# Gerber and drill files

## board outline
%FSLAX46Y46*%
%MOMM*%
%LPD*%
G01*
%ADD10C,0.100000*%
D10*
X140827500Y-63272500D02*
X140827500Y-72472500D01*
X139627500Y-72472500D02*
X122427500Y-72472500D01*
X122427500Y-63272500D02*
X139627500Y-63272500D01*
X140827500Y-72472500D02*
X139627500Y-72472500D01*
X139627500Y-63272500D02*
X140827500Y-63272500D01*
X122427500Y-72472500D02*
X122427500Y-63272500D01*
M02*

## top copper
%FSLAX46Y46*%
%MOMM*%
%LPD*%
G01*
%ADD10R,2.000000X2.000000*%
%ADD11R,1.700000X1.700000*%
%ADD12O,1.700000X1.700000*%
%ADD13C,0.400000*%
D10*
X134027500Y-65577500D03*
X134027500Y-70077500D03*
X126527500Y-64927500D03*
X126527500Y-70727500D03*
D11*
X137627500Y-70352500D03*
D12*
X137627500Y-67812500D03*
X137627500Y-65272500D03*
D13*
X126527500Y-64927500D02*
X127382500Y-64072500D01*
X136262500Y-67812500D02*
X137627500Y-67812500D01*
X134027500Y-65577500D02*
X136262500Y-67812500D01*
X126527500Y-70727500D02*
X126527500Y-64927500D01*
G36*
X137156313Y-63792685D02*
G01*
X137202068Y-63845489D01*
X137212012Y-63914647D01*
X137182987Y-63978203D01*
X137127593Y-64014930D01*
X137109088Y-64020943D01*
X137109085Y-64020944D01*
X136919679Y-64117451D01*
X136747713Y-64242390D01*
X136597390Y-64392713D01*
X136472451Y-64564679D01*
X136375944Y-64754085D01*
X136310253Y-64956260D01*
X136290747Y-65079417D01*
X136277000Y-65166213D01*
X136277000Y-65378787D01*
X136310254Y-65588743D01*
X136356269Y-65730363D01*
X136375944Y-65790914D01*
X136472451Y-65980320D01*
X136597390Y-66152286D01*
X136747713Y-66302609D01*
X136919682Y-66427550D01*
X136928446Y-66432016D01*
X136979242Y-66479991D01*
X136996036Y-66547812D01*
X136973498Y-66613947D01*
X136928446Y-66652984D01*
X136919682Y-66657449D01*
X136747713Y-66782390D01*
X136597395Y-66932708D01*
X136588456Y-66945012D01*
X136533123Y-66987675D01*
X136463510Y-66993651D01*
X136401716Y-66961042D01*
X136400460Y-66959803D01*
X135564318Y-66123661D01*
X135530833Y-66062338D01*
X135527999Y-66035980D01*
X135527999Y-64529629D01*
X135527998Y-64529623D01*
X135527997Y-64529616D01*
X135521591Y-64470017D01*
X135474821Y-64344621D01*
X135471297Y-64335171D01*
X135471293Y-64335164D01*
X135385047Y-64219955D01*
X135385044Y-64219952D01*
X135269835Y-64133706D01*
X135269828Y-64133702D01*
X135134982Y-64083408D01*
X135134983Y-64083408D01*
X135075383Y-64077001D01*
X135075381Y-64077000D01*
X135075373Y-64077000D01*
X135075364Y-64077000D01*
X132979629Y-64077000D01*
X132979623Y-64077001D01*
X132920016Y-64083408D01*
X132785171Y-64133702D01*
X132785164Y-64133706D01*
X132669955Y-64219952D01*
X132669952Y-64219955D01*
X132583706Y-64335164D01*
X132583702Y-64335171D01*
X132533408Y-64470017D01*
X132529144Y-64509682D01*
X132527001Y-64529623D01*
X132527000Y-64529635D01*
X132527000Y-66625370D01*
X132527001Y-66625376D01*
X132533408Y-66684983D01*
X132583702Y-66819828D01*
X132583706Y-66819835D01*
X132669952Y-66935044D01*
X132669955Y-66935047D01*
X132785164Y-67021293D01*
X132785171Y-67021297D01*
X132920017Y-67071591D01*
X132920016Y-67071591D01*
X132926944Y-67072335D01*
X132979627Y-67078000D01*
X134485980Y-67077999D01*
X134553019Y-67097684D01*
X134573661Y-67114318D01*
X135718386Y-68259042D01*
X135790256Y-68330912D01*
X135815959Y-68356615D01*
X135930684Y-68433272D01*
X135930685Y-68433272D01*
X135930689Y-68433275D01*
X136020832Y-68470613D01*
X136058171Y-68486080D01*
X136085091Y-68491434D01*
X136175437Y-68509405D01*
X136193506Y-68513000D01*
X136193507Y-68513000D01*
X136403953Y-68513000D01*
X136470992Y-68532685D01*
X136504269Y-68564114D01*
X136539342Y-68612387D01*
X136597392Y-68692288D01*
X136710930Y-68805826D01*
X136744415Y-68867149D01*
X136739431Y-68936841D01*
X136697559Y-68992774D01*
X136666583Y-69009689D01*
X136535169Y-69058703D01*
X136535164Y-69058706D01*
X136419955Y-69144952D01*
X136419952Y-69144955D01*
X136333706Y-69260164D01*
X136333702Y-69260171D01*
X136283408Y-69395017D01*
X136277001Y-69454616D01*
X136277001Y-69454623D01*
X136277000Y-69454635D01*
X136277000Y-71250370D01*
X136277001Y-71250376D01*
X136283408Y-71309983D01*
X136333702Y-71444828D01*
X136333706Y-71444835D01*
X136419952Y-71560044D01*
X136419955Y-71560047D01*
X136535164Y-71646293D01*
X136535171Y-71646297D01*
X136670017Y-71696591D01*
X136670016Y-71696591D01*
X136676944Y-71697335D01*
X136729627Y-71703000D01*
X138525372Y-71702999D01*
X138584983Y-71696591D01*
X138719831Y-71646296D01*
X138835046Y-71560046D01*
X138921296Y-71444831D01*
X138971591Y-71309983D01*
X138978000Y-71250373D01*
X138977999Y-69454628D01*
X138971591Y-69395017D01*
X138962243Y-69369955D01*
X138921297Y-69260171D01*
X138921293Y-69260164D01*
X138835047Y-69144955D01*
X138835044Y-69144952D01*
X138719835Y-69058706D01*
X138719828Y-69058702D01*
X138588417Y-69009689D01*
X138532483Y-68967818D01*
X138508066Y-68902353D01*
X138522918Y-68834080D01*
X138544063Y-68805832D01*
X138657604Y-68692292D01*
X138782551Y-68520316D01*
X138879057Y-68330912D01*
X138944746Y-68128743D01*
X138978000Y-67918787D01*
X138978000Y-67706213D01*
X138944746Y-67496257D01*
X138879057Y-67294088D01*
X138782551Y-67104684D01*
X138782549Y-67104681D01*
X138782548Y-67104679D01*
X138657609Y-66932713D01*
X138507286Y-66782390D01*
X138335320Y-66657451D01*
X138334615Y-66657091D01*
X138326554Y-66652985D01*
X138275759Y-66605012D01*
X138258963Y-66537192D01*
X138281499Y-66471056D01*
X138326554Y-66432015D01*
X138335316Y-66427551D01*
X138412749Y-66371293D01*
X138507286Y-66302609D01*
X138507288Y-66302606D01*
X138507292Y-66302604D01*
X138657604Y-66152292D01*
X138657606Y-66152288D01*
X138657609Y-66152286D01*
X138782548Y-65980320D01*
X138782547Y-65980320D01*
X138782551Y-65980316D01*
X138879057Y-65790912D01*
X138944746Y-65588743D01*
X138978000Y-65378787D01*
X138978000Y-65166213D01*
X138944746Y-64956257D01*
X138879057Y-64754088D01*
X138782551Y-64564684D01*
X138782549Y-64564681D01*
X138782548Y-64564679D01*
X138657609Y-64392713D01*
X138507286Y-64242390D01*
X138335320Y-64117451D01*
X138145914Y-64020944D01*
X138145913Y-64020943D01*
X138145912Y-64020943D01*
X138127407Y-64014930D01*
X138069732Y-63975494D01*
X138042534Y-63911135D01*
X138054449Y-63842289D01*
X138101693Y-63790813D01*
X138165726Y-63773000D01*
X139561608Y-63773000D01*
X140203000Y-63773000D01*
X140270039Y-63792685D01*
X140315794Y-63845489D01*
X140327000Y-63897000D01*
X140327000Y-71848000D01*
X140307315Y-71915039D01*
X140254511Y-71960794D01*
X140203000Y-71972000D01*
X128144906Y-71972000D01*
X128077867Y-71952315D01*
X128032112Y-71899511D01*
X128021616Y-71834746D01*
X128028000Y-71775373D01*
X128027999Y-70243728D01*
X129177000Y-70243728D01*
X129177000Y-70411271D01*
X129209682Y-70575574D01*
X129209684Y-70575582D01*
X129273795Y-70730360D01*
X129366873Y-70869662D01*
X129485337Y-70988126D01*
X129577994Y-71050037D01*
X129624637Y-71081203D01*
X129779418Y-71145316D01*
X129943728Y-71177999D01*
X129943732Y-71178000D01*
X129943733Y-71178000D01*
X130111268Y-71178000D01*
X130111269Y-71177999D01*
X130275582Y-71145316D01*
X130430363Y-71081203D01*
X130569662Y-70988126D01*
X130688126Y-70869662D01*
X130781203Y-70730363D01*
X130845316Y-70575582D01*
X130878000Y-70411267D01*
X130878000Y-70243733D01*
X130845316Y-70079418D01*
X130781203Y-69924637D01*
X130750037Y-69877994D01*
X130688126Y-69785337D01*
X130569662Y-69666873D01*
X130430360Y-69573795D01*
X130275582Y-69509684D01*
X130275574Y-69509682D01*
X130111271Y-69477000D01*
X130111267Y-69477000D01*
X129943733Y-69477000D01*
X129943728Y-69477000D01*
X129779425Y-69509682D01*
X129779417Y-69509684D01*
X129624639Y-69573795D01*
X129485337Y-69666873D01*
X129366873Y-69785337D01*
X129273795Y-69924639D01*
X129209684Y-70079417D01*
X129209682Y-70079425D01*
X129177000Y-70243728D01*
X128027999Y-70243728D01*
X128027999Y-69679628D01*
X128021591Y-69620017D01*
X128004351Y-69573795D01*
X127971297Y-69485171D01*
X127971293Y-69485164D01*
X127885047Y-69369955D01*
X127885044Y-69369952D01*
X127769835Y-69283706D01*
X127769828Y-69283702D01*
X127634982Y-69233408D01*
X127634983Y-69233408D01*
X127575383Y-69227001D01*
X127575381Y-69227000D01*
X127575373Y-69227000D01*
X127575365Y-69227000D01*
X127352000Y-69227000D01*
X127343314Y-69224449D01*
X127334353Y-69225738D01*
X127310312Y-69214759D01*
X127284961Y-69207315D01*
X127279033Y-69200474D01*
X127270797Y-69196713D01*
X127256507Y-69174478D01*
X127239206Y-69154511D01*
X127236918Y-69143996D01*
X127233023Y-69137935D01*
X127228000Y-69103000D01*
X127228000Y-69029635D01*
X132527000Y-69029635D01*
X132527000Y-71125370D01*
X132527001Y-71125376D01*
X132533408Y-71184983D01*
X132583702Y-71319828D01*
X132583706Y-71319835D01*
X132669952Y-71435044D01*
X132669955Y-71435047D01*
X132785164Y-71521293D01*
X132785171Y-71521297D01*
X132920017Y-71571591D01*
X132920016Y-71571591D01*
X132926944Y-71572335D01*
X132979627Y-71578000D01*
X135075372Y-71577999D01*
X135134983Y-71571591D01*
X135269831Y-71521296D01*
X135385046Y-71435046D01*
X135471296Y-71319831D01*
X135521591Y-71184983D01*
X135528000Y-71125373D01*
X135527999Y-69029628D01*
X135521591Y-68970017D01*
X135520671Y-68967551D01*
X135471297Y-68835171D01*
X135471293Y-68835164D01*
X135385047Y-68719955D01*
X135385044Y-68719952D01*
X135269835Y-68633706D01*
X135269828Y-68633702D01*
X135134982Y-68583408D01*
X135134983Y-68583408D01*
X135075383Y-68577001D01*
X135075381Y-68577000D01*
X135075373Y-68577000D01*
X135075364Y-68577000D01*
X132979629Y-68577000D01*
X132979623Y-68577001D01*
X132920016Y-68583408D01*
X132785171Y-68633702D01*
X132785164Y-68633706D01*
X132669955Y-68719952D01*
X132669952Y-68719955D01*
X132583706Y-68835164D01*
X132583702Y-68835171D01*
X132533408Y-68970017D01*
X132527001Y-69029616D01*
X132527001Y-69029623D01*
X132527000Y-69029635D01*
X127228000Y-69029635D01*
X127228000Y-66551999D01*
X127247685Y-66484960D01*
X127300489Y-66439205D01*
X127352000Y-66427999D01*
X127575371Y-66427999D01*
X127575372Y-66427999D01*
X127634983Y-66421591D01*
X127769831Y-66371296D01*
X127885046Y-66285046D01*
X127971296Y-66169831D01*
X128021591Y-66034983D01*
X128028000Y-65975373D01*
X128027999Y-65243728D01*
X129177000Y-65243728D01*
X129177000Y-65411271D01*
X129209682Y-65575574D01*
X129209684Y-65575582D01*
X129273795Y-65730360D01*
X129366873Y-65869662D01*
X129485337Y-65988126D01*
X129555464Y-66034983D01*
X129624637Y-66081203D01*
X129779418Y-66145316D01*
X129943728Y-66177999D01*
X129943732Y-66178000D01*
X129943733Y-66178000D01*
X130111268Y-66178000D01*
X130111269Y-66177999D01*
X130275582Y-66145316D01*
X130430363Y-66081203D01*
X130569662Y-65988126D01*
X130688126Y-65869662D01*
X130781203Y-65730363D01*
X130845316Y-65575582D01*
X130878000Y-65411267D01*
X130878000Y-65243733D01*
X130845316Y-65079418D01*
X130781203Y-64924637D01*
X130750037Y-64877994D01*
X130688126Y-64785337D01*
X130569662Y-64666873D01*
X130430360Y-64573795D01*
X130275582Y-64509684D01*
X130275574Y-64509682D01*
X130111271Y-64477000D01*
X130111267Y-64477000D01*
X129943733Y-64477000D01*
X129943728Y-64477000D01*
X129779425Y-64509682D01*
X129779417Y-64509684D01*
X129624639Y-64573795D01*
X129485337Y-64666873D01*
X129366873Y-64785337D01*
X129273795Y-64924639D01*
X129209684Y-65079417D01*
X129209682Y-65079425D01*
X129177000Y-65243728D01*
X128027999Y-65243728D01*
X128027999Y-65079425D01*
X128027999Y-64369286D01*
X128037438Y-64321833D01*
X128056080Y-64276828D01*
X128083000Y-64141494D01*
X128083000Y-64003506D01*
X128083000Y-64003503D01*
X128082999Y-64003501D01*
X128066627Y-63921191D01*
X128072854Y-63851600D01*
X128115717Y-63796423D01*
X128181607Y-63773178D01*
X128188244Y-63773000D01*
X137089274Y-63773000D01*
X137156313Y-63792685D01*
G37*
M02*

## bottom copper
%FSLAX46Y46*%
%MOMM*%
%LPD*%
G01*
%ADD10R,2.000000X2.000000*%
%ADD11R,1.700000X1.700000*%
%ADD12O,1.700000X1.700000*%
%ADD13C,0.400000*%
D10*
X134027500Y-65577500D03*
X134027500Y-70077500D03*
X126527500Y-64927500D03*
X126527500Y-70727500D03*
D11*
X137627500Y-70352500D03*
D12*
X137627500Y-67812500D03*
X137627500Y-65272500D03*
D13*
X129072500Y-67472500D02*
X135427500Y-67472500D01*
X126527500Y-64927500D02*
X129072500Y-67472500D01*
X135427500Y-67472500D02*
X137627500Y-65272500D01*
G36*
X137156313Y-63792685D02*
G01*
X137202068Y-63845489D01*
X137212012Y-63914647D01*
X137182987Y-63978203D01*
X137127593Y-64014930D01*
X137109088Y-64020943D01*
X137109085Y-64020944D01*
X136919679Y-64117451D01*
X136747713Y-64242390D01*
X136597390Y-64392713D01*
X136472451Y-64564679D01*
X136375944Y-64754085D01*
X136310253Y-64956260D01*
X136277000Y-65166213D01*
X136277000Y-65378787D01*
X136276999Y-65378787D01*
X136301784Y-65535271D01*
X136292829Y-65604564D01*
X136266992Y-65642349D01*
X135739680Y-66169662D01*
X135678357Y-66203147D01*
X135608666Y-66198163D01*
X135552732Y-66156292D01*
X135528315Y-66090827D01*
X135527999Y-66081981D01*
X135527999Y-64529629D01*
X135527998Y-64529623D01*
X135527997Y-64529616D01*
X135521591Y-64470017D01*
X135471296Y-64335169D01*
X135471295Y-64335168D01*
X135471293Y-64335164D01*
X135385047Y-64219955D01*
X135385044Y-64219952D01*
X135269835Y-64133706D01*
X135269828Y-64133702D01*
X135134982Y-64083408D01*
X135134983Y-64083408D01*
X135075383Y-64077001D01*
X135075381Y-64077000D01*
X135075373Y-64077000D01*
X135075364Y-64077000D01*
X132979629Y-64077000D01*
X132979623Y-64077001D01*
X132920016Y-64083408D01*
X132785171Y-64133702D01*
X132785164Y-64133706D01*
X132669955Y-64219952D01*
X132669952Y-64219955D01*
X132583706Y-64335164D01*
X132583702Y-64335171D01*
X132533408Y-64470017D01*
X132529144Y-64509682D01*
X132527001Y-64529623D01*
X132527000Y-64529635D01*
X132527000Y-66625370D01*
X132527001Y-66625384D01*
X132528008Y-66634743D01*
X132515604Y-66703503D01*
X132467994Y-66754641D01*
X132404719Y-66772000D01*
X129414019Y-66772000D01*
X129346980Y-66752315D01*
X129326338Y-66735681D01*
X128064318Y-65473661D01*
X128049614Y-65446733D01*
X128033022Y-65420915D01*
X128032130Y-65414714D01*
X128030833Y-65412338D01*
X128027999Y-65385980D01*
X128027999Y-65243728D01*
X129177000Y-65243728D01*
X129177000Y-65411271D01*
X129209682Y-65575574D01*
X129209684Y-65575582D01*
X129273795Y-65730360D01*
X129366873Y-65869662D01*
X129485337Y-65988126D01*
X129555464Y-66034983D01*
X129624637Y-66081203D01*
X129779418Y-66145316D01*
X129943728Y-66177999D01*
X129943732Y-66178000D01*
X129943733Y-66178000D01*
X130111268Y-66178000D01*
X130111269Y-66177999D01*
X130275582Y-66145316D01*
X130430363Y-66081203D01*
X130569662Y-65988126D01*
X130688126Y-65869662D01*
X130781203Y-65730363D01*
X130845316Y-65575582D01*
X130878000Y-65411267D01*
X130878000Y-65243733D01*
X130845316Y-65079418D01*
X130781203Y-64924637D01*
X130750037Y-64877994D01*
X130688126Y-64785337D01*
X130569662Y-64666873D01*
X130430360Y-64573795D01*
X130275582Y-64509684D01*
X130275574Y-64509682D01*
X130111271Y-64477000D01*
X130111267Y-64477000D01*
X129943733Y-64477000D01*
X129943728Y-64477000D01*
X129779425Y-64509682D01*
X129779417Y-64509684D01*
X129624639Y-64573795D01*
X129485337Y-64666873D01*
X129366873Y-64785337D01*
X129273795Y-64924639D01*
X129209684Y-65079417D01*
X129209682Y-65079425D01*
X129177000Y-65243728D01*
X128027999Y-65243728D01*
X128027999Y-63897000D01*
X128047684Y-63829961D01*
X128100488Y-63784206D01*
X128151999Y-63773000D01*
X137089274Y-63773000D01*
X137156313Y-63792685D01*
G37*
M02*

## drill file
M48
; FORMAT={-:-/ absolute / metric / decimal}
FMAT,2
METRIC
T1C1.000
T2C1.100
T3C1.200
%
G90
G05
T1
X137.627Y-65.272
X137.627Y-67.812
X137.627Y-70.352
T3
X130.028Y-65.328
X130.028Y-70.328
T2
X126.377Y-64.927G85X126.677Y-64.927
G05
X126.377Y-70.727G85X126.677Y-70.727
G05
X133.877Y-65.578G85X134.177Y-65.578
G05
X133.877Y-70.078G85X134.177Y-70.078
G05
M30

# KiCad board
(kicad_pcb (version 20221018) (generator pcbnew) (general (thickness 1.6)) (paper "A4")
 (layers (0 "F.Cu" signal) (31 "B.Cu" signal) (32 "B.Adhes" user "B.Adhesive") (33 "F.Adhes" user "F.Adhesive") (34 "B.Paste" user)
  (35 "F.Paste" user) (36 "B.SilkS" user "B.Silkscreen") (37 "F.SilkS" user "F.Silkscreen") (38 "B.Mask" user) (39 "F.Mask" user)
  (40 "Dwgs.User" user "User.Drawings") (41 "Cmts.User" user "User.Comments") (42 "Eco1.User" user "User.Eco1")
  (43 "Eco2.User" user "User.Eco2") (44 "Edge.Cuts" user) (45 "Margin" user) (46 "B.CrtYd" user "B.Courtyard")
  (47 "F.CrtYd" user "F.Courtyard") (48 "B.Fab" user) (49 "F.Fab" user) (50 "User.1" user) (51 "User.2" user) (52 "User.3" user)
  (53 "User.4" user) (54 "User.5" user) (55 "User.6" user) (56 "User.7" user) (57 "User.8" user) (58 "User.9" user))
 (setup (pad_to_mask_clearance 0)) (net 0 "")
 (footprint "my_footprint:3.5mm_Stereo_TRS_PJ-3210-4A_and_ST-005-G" (layer "F.Cu") (at 123.0275 67.8275)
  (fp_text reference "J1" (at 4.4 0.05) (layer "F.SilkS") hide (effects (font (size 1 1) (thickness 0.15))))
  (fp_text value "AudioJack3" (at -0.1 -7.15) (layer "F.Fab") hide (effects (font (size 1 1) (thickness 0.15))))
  (pad "" np_thru_hole circle (at 7 -2.5) (size 1.2 1.2) (drill 1.2) (layers "*.Cu" "*.Mask"))
  (pad "" np_thru_hole circle (at 7 2.5) (size 1.2 1.2) (drill 1.2) (layers "*.Cu" "*.Mask"))
  (pad "R" thru_hole rect (at 11 -2.25) (size 2 2) (drill oval 1.4 1.1) (layers "*.Cu" "*.Mask"))
  (pad "S" thru_hole rect (at 11 2.25) (size 2 2) (drill oval 1.4 1.1) (layers "*.Cu" "*.Mask"))
  (pad "T" thru_hole rect (at 3.5 -2.9) (size 2 2) (drill oval 1.4 1.1) (layers "*.Cu" "*.Mask"))
  (pad "T" thru_hole rect (at 3.5 2.9) (size 2 2) (drill oval 1.4 1.1) (layers "*.Cu" "*.Mask")))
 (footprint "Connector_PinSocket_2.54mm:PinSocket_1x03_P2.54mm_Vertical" (layer "F.Cu") (at 137.6275 70.3525 180)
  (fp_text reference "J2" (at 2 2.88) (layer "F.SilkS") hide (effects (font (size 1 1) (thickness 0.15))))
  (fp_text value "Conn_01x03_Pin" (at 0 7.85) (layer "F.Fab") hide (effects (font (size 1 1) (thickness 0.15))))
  (pad "1" thru_hole rect (at 0 0 180) (size 1.7 1.7) (drill 1) (layers "*.Cu" "*.Mask"))
  (pad "2" thru_hole oval (at 0 2.54 180) (size 1.7 1.7) (drill 1) (layers "*.Cu" "*.Mask"))
  (pad "3" thru_hole oval (at 0 5.08 180) (size 1.7 1.7) (drill 1) (layers "*.Cu" "*.Mask")))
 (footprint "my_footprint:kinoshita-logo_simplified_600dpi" (layer "B.Cu") (at 130.4275 67.8198 -90)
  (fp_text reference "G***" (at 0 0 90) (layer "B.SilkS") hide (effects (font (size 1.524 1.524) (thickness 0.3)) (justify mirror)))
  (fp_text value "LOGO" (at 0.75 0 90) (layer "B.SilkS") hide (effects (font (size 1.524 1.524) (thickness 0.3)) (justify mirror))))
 (gr_line (start 140.8275 63.2725) (end 140.8275 72.4725) (stroke (width 0.1) (type default)) (layer "Edge.Cuts"))
 (gr_line (start 139.6275 72.4725) (end 122.4275 72.4725) (stroke (width 0.1) (type default)) (layer "Edge.Cuts"))
 (gr_line (start 122.4275 63.2725) (end 139.6275 63.2725) (stroke (width 0.1) (type default)) (layer "Edge.Cuts"))
 (gr_line (start 140.8275 72.4725) (end 139.6275 72.4725) (stroke (width 0.1) (type default)) (layer "Edge.Cuts"))
 (gr_line (start 139.6275 63.2725) (end 140.8275 63.2725) (stroke (width 0.1) (type default)) (layer "Edge.Cuts"))
 (gr_line (start 122.4275 72.4725) (end 122.4275 63.2725) (stroke (width 0.1) (type default)) (layer "Edge.Cuts"))
 (segment (start 126.5275 64.9275) (end 127.3825 64.0725) (width 0.4) (layer "F.Cu") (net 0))
 (segment (start 136.2625 67.8125) (end 137.6275 67.8125) (width 0.4) (layer "F.Cu") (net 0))
 (segment (start 134.0275 65.5775) (end 136.2625 67.8125) (width 0.4) (layer "F.Cu") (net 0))
 (segment (start 126.5275 70.7275) (end 126.5275 64.9275) (width 0.4) (layer "F.Cu") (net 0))
 (segment (start 129.0725 67.4725) (end 135.4275 67.4725) (width 0.4) (layer "B.Cu") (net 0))
 (segment (start 126.5275 64.9275) (end 129.0725 67.4725) (width 0.4) (layer "B.Cu") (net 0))
 (segment (start 135.4275 67.4725) (end 137.6275 65.2725) (width 0.4) (layer "B.Cu") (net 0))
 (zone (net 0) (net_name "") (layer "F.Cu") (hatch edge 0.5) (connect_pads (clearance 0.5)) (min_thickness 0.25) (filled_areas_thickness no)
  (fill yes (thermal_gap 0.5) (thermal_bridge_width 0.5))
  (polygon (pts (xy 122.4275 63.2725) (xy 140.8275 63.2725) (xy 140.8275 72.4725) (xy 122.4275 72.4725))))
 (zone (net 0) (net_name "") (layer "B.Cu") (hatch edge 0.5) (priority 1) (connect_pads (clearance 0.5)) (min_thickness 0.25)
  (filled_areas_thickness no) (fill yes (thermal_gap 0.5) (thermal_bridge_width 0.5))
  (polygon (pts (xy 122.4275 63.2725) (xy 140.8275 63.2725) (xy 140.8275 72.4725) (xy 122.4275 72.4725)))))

